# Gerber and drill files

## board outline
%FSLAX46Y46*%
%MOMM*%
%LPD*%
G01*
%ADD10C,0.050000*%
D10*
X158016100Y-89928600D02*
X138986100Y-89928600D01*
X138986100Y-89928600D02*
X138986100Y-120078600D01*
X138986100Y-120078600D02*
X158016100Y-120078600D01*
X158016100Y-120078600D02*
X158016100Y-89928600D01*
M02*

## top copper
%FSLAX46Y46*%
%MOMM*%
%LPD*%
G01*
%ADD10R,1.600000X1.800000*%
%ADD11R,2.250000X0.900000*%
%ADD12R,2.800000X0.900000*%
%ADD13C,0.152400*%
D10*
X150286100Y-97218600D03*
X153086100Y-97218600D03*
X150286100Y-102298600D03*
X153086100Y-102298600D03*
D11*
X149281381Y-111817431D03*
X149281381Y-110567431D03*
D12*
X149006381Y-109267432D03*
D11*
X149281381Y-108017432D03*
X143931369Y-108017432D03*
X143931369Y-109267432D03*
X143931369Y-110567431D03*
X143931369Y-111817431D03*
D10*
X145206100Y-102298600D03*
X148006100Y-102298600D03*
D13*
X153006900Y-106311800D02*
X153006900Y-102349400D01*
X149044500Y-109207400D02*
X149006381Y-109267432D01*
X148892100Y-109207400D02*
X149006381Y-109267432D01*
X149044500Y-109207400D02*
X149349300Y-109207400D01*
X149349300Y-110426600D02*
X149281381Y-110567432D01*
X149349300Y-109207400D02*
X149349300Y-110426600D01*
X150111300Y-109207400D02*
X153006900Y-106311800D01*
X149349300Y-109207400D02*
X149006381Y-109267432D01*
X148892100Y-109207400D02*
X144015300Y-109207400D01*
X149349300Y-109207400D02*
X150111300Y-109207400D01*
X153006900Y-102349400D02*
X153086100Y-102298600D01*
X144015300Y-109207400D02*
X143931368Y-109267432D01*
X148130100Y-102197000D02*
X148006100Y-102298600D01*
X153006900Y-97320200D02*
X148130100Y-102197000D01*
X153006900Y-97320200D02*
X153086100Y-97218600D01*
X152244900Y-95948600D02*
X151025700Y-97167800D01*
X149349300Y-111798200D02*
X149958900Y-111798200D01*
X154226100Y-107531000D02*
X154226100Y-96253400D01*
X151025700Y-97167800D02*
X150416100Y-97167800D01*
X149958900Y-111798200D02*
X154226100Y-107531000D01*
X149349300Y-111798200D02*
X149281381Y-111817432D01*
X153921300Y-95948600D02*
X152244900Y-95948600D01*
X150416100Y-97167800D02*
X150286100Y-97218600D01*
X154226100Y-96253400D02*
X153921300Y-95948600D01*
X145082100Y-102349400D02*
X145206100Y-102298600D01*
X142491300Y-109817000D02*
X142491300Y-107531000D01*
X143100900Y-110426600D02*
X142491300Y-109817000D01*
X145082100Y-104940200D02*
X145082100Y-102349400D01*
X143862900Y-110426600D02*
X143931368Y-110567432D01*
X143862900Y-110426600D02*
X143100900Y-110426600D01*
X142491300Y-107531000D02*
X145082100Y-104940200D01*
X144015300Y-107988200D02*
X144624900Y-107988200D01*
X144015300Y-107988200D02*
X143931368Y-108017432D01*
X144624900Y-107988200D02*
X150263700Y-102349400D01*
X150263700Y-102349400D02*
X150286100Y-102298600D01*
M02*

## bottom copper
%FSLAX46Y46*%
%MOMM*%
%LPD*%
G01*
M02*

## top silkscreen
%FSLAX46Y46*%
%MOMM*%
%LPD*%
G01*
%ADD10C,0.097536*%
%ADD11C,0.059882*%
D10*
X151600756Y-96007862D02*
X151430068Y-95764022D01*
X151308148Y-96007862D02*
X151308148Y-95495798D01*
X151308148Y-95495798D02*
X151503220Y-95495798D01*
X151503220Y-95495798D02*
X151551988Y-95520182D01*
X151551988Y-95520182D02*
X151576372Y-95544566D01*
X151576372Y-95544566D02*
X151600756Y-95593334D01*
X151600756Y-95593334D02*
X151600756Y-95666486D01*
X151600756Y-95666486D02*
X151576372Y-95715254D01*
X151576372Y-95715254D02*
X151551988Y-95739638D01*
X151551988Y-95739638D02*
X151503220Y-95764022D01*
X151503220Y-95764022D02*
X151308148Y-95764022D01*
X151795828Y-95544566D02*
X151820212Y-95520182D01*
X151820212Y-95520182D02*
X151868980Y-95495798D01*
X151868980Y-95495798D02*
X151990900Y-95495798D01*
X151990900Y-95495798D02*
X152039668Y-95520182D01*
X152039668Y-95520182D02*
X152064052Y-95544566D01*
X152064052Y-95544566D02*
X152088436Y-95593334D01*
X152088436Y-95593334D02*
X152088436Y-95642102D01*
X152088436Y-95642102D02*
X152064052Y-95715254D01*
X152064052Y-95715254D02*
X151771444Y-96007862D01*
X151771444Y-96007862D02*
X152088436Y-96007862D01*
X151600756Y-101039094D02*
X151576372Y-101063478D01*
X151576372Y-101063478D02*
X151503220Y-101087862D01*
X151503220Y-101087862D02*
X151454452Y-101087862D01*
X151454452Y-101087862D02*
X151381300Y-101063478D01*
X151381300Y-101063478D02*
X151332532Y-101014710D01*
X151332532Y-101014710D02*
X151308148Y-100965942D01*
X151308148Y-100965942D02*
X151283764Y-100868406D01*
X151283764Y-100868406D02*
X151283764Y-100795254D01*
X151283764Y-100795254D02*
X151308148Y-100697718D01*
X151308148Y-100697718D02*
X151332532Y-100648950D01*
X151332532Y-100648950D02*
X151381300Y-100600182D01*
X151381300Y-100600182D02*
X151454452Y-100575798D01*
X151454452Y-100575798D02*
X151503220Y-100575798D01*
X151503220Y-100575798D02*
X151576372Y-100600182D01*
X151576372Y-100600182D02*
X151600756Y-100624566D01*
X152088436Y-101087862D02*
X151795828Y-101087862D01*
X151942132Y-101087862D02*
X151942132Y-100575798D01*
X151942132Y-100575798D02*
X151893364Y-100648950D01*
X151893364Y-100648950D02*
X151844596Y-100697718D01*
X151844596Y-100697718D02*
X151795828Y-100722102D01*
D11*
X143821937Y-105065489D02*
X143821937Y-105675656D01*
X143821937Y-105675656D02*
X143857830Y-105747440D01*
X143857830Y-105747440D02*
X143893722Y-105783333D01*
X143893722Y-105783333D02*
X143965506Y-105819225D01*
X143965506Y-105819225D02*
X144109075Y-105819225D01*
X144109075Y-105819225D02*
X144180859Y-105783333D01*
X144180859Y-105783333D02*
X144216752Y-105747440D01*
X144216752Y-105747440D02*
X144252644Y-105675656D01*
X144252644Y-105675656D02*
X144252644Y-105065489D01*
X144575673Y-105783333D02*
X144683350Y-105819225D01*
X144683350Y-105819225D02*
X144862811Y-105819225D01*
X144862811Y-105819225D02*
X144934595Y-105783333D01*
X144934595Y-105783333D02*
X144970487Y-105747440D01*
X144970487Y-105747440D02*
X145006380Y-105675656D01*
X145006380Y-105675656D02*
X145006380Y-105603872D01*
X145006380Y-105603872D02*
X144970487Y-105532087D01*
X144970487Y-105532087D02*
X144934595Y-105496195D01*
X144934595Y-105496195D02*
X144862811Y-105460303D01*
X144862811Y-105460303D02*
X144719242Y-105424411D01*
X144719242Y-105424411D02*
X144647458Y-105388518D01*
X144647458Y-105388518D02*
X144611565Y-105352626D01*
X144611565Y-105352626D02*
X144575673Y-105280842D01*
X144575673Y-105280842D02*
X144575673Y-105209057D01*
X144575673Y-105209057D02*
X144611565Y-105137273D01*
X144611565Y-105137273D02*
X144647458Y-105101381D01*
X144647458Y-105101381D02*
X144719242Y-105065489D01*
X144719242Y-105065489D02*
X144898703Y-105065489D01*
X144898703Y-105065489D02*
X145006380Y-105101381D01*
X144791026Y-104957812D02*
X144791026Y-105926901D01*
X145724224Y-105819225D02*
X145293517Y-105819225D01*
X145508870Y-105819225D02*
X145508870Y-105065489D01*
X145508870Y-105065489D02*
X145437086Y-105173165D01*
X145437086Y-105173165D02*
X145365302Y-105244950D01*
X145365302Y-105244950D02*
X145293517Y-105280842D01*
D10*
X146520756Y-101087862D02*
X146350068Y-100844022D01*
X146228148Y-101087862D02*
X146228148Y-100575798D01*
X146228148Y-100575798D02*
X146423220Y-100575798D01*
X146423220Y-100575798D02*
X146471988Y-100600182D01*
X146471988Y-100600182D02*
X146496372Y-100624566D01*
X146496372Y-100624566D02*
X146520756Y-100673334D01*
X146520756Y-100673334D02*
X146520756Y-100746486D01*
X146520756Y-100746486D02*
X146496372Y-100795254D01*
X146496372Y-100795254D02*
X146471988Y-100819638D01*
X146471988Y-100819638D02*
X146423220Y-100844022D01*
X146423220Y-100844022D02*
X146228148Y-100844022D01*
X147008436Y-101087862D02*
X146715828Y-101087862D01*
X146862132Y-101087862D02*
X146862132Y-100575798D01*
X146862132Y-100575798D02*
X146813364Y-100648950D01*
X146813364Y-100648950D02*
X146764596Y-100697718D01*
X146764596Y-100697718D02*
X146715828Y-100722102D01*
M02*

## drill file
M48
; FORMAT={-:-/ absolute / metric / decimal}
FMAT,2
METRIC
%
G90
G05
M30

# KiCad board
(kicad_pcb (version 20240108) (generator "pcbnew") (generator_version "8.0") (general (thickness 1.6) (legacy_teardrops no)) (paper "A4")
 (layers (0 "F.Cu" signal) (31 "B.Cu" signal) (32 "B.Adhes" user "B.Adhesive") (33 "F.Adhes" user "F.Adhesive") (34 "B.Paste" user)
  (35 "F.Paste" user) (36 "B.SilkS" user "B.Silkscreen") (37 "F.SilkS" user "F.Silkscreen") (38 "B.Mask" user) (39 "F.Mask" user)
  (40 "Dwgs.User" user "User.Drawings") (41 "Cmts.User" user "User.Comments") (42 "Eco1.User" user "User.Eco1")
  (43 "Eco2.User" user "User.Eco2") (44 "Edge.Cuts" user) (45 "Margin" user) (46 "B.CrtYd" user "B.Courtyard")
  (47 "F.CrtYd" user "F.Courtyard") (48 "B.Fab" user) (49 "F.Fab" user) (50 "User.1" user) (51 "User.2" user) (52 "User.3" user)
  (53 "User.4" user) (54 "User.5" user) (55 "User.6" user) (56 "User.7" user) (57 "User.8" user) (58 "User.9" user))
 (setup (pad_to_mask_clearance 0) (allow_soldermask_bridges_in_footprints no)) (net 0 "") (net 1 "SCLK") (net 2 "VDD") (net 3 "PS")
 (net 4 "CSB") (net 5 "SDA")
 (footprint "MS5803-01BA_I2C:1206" (layer "F.Cu") (at 151.6861 97.2186)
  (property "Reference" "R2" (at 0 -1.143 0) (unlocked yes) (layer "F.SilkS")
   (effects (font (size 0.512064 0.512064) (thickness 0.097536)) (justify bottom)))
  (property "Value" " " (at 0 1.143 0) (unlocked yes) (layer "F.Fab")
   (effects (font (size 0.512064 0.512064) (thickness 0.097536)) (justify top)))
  (pad "1" smd rect (at -1.4 0) (size 1.6 1.8) (layers "F.Cu" "F.Paste" "F.Mask") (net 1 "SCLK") (solder_mask_margin 0.1016)
   (thermal_bridge_angle 0))
  (pad "2" smd rect (at 1.4 0) (size 1.6 1.8) (layers "F.Cu" "F.Paste" "F.Mask") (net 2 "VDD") (solder_mask_margin 0.1016)
   (thermal_bridge_angle 0)))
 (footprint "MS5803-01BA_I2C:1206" (layer "F.Cu") (at 151.6861 102.2986)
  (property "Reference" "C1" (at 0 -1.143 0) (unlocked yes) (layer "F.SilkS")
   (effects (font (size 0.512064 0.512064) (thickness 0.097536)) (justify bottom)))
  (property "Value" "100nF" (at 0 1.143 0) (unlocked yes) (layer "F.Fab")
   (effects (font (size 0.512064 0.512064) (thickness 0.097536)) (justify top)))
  (pad "1" smd rect (at -1.4 0) (size 1.6 1.8) (layers "F.Cu" "F.Paste" "F.Mask") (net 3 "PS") (solder_mask_margin 0.1016)
   (thermal_bridge_angle 0))
  (pad "2" smd rect (at 1.4 0) (size 1.6 1.8) (layers "F.Cu" "F.Paste" "F.Mask") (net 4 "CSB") (solder_mask_margin 0.1016)
   (thermal_bridge_angle 0)))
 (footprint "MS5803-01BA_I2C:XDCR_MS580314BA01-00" (layer "F.Cu") (at 146.6061 109.9186)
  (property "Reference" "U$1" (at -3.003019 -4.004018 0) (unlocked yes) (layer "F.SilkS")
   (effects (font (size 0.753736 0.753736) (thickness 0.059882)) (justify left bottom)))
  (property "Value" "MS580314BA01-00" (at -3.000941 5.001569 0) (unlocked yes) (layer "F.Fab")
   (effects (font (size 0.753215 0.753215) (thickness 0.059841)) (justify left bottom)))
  (pad "1" smd rect (at 2.675281 1.898831) (size 2.25 0.9) (layers "F.Cu" "F.Paste" "F.Mask") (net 1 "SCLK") (solder_mask_margin 0.1016)
   (thermal_bridge_angle 0))
  (pad "2" smd rect (at 2.675281 0.648831) (size 2.25 0.9) (layers "F.Cu" "F.Paste" "F.Mask") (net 4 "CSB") (solder_mask_margin 0.1016)
   (thermal_bridge_angle 0))
  (pad "3" smd rect (at 2.400281 -0.651168) (size 2.8 0.9) (layers "F.Cu" "F.Paste" "F.Mask") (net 4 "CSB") (solder_mask_margin 0.1016)
   (thermal_bridge_angle 0))
  (pad "4" smd rect (at 2.675281 -1.901168) (size 2.25 0.9) (layers "F.Cu" "F.Paste" "F.Mask") (solder_mask_margin 0.1016)
   (thermal_bridge_angle 0))
  (pad "5" smd rect (at -2.674731 -1.901168) (size 2.25 0.9) (layers "F.Cu" "F.Paste" "F.Mask") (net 3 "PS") (solder_mask_margin 0.1016)
   (thermal_bridge_angle 0))
  (pad "6" smd rect (at -2.674731 -0.651168) (size 2.25 0.9) (layers "F.Cu" "F.Paste" "F.Mask") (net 4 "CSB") (solder_mask_margin 0.1016)
   (thermal_bridge_angle 0))
  (pad "7" smd rect (at -2.674731 0.648831) (size 2.25 0.9) (layers "F.Cu" "F.Paste" "F.Mask") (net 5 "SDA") (solder_mask_margin 0.1016)
   (thermal_bridge_angle 0))
  (pad "8" smd rect (at -2.674731 1.898831) (size 2.25 0.9) (layers "F.Cu" "F.Paste" "F.Mask") (solder_mask_margin 0.1016)
   (thermal_bridge_angle 0)))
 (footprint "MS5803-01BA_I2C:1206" (layer "F.Cu") (at 146.6061 102.2986)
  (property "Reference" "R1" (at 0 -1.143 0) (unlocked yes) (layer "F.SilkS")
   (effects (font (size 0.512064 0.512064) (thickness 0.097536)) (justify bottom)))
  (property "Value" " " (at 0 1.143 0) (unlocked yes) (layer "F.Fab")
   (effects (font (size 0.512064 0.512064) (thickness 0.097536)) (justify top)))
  (pad "1" smd rect (at -1.4 0) (size 1.6 1.8) (layers "F.Cu" "F.Paste" "F.Mask") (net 5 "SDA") (solder_mask_margin 0.1016)
   (thermal_bridge_angle 0))
  (pad "2" smd rect (at 1.4 0) (size 1.6 1.8) (layers "F.Cu" "F.Paste" "F.Mask") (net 2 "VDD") (solder_mask_margin 0.1016)
   (thermal_bridge_angle 0)))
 (gr_line (start 158.0161 89.9286) (end 138.9861 89.9286) (stroke (width 0.05) (type solid)) (layer "Edge.Cuts"))
 (gr_line (start 138.9861 89.9286) (end 138.9861 120.0786) (stroke (width 0.05) (type solid)) (layer "Edge.Cuts"))
 (gr_line (start 138.9861 120.0786) (end 158.0161 120.0786) (stroke (width 0.05) (type solid)) (layer "Edge.Cuts"))
 (gr_line (start 158.0161 120.0786) (end 158.0161 89.9286) (stroke (width 0.05) (type solid)) (layer "Edge.Cuts"))
 (segment (start 153.0069 106.3118) (end 153.0069 102.3494) (width 0.1524) (layer "F.Cu") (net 4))
 (segment (start 149.0445 109.2074) (end 149.006381 109.267432) (width 0.1524) (layer "F.Cu") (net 4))
 (segment (start 148.8921 109.2074) (end 149.006381 109.267432) (width 0.1524) (layer "F.Cu") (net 4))
 (segment (start 149.0445 109.2074) (end 149.3493 109.2074) (width 0.1524) (layer "F.Cu") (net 4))
 (segment (start 149.3493 110.4266) (end 149.281381 110.567432) (width 0.1524) (layer "F.Cu") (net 4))
 (segment (start 149.3493 109.2074) (end 149.3493 110.4266) (width 0.1524) (layer "F.Cu") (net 4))
 (segment (start 150.1113 109.2074) (end 153.0069 106.3118) (width 0.1524) (layer "F.Cu") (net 4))
 (segment (start 149.3493 109.2074) (end 149.006381 109.267432) (width 0.1524) (layer "F.Cu") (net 4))
 (segment (start 148.8921 109.2074) (end 144.0153 109.2074) (width 0.1524) (layer "F.Cu") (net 4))
 (segment (start 149.3493 109.2074) (end 150.1113 109.2074) (width 0.1524) (layer "F.Cu") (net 4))
 (segment (start 153.0069 102.3494) (end 153.0861 102.2986) (width 0.1524) (layer "F.Cu") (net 4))
 (segment (start 144.0153 109.2074) (end 143.931368 109.267432) (width 0.1524) (layer "F.Cu") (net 4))
 (segment (start 148.1301 102.197) (end 148.0061 102.2986) (width 0.1524) (layer "F.Cu") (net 2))
 (segment (start 153.0069 97.3202) (end 148.1301 102.197) (width 0.1524) (layer "F.Cu") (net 2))
 (segment (start 153.0069 97.3202) (end 153.0861 97.2186) (width 0.1524) (layer "F.Cu") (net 2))
 (segment (start 152.2449 95.9486) (end 151.0257 97.1678) (width 0.1524) (layer "F.Cu") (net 1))
 (segment (start 149.3493 111.7982) (end 149.9589 111.7982) (width 0.1524) (layer "F.Cu") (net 1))
 (segment (start 154.2261 107.531) (end 154.2261 96.2534) (width 0.1524) (layer "F.Cu") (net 1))
 (segment (start 151.0257 97.1678) (end 150.4161 97.1678) (width 0.1524) (layer "F.Cu") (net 1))
 (segment (start 149.9589 111.7982) (end 154.2261 107.531) (width 0.1524) (layer "F.Cu") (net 1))
 (segment (start 149.3493 111.7982) (end 149.281381 111.817432) (width 0.1524) (layer "F.Cu") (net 1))
 (segment (start 153.9213 95.9486) (end 152.2449 95.9486) (width 0.1524) (layer "F.Cu") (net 1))
 (segment (start 150.4161 97.1678) (end 150.2861 97.2186) (width 0.1524) (layer "F.Cu") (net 1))
 (segment (start 154.2261 96.2534) (end 153.9213 95.9486) (width 0.1524) (layer "F.Cu") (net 1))
 (segment (start 145.0821 102.3494) (end 145.2061 102.2986) (width 0.1524) (layer "F.Cu") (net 5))
 (segment (start 142.4913 109.817) (end 142.4913 107.531) (width 0.1524) (layer "F.Cu") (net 5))
 (segment (start 143.1009 110.4266) (end 142.4913 109.817) (width 0.1524) (layer "F.Cu") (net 5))
 (segment (start 145.0821 104.9402) (end 145.0821 102.3494) (width 0.1524) (layer "F.Cu") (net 5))
 (segment (start 143.8629 110.4266) (end 143.931368 110.567432) (width 0.1524) (layer "F.Cu") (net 5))
 (segment (start 143.8629 110.4266) (end 143.1009 110.4266) (width 0.1524) (layer "F.Cu") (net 5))
 (segment (start 142.4913 107.531) (end 145.0821 104.9402) (width 0.1524) (layer "F.Cu") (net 5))
 (segment (start 144.0153 107.9882) (end 144.6249 107.9882) (width 0.1524) (layer "F.Cu") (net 3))
 (segment (start 144.0153 107.9882) (end 143.931368 108.017432) (width 0.1524) (layer "F.Cu") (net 3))
 (segment (start 144.6249 107.9882) (end 150.2637 102.3494) (width 0.1524) (layer "F.Cu") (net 3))
 (segment (start 150.2637 102.3494) (end 150.2861 102.2986) (width 0.1524) (layer "F.Cu") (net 3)))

